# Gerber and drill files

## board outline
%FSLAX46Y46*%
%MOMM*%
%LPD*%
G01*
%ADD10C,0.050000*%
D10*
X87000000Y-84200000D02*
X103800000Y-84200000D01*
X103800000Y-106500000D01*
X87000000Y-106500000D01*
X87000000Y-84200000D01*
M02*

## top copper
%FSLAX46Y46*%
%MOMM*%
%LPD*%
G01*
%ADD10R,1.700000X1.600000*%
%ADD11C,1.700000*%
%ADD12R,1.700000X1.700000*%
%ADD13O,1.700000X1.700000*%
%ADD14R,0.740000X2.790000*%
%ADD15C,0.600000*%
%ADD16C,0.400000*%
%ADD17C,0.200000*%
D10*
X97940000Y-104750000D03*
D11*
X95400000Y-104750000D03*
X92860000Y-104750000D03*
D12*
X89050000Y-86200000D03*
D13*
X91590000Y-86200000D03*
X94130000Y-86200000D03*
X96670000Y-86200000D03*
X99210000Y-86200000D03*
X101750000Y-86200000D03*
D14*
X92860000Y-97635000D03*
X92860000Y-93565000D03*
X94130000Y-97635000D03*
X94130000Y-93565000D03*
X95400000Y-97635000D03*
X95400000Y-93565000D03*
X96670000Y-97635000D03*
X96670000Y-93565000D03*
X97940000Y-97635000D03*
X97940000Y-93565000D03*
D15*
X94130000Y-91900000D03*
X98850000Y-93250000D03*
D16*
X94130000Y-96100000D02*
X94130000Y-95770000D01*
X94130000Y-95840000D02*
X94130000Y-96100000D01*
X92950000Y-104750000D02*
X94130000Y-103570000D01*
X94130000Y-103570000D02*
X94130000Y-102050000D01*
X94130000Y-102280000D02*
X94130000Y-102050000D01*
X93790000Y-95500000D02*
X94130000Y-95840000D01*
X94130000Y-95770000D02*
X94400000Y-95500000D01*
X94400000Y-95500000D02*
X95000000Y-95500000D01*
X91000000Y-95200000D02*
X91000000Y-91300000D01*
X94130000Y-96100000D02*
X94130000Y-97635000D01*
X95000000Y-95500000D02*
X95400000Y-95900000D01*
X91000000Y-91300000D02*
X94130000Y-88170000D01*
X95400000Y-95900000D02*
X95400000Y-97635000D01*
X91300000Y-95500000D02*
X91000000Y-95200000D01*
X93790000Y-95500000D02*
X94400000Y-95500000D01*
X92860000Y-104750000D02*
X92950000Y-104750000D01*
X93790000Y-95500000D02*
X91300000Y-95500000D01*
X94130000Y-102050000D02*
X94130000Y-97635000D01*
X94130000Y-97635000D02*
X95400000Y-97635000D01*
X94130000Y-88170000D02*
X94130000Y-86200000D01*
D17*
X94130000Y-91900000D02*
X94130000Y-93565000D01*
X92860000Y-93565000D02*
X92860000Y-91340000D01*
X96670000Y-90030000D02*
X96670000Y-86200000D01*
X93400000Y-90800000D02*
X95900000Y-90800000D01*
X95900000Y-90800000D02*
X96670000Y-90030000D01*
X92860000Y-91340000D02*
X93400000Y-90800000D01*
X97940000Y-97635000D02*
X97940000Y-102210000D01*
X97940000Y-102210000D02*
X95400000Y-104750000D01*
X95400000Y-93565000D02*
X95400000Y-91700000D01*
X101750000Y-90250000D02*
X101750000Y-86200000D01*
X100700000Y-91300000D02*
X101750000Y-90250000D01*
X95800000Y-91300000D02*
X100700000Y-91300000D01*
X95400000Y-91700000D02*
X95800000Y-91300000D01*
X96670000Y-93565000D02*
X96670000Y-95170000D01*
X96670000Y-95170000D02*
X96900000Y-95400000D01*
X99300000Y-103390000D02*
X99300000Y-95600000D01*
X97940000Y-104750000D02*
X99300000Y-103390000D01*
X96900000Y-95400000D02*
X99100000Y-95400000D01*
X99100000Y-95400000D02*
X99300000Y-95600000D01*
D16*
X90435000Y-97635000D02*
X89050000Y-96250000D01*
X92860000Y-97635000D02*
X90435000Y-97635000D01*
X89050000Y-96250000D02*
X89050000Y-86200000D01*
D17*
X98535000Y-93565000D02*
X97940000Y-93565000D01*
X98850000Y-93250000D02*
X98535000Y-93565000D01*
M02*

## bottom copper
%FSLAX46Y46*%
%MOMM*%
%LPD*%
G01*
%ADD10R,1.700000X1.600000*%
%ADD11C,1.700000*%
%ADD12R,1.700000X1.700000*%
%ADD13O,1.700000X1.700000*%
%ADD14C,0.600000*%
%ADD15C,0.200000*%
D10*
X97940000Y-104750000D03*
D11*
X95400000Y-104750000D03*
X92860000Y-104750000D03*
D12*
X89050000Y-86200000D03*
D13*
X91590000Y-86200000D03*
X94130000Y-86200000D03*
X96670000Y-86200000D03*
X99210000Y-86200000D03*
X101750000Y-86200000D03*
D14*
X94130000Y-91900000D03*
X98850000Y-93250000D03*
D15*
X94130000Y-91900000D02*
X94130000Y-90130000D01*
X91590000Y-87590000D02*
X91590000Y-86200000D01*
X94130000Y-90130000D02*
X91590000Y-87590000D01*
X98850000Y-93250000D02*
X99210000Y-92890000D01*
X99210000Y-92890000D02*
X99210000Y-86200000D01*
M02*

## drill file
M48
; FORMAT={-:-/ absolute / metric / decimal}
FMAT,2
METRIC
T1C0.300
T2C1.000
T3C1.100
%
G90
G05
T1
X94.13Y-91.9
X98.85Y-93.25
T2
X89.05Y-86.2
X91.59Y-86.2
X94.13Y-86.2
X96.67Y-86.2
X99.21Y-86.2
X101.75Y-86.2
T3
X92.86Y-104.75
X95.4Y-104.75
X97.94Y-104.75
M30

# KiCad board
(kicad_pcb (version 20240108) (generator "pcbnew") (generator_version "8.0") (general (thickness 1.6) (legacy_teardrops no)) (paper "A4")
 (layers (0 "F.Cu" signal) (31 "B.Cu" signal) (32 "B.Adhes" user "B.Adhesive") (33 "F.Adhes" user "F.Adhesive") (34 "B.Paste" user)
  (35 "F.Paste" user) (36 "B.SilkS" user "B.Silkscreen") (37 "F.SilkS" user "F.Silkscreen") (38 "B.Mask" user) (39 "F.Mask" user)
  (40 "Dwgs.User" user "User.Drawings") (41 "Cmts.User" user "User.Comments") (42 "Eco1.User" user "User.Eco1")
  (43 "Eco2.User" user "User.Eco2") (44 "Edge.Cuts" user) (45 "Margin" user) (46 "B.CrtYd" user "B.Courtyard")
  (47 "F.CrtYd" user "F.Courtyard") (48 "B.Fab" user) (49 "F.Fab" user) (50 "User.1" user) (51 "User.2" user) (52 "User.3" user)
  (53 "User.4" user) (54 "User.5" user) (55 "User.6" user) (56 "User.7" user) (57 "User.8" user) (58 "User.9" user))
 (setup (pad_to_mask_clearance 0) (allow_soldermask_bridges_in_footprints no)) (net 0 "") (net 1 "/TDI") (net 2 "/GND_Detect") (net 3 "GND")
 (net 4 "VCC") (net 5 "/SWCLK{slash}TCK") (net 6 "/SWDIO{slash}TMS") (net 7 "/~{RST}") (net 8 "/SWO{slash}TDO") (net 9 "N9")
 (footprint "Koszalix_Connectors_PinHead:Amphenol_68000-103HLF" (layer "F.Cu") (at 95.4 104.75 180)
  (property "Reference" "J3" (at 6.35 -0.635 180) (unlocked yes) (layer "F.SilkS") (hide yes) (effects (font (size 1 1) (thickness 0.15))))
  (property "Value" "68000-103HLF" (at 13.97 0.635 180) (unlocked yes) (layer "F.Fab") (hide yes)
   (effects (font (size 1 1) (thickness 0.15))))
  (pad "1" thru_hole rect (at -2.54 0 180) (size 1.7 1.6) (drill 1.1) (layers "*.Cu" "*.Mask") (remove_unused_layers no) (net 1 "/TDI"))
  (pad "2" thru_hole circle (at 0 0 180) (size 1.7 1.7) (drill 1.1) (layers "*.Cu" "*.Mask") (remove_unused_layers no) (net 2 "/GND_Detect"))
  (pad "3" thru_hole circle (at 2.54 0 180) (size 1.7 1.7) (drill 1.1) (layers "*.Cu" "*.Mask") (remove_unused_layers no) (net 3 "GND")))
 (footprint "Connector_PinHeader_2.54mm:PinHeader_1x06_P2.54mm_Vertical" (layer "F.Cu") (at 89.05 86.2 90)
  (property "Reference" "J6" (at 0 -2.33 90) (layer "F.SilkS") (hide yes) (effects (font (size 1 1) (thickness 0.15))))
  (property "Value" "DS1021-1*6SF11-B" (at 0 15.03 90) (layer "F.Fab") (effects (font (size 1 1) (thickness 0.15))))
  (pad "1" thru_hole rect (at 0 0 90) (size 1.7 1.7) (drill 1) (layers "*.Cu" "*.Mask") (remove_unused_layers no) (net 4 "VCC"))
  (pad "2" thru_hole oval (at 0 2.54 90) (size 1.7 1.7) (drill 1) (layers "*.Cu" "*.Mask") (remove_unused_layers no)
   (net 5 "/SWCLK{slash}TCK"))
  (pad "3" thru_hole oval (at 0 5.08 90) (size 1.7 1.7) (drill 1) (layers "*.Cu" "*.Mask") (remove_unused_layers no) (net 3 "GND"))
  (pad "4" thru_hole oval (at 0 7.62 90) (size 1.7 1.7) (drill 1) (layers "*.Cu" "*.Mask") (remove_unused_layers no)
   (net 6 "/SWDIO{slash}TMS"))
  (pad "5" thru_hole oval (at 0 10.16 90) (size 1.7 1.7) (drill 1) (layers "*.Cu" "*.Mask") (remove_unused_layers no) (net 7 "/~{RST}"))
  (pad "6" thru_hole oval (at 0 12.7 90) (size 1.7 1.7) (drill 1) (layers "*.Cu" "*.Mask") (remove_unused_layers no)
   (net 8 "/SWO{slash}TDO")))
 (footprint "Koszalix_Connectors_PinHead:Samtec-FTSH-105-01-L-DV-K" (layer "F.Cu") (at 95.4 95.6)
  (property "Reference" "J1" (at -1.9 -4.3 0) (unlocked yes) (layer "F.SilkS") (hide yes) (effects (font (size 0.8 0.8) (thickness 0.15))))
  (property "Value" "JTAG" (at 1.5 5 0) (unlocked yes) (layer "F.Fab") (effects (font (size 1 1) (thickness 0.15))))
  (pad "1" smd rect (at -2.54 2.035) (size 0.74 2.79) (layers "F.Cu" "F.Paste" "F.Mask") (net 4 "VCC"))
  (pad "2" smd rect (at -2.54 -2.035) (size 0.74 2.79) (layers "F.Cu" "F.Paste" "F.Mask") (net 6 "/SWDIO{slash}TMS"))
  (pad "3" smd rect (at -1.27 2.035) (size 0.74 2.79) (layers "F.Cu" "F.Paste" "F.Mask") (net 3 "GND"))
  (pad "4" smd rect (at -1.27 -2.035) (size 0.74 2.79) (layers "F.Cu" "F.Paste" "F.Mask") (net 5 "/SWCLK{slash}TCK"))
  (pad "5" smd rect (at 0 2.035) (size 0.74 2.79) (layers "F.Cu" "F.Paste" "F.Mask") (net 3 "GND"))
  (pad "6" smd rect (at 0 -2.035) (size 0.74 2.79) (layers "F.Cu" "F.Paste" "F.Mask") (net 8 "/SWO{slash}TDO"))
  (pad "7" smd rect (at 1.27 2.035) (size 0.74 2.79) (layers "F.Cu" "F.Paste" "F.Mask") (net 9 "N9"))
  (pad "8" smd rect (at 1.27 -2.035) (size 0.74 2.79) (layers "F.Cu" "F.Paste" "F.Mask") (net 1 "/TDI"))
  (pad "9" smd rect (at 2.54 2.035) (size 0.74 2.79) (layers "F.Cu" "F.Paste" "F.Mask") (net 2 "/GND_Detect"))
  (pad "10" smd rect (at 2.54 -2.035) (size 0.74 2.79) (layers "F.Cu" "F.Paste" "F.Mask") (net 7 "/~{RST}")))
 (gr_rect (start 87 84.2) (end 103.8 106.5) (stroke (width 0.05) (type default)) (fill none) (layer "Edge.Cuts"))
 (segment (start 94.13 96.1) (end 94.13 95.77) (width 0.4) (layer "F.Cu") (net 3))
 (segment (start 94.13 95.84) (end 94.13 96.1) (width 0.4) (layer "F.Cu") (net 3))
 (segment (start 92.95 104.75) (end 94.13 103.57) (width 0.4) (layer "F.Cu") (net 3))
 (segment (start 94.13 103.57) (end 94.13 102.05) (width 0.4) (layer "F.Cu") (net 3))
 (segment (start 94.13 102.28) (end 94.13 102.05) (width 0.4) (layer "F.Cu") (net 3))
 (segment (start 93.79 95.5) (end 94.13 95.84) (width 0.4) (layer "F.Cu") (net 3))
 (segment (start 94.13 95.77) (end 94.4 95.5) (width 0.4) (layer "F.Cu") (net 3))
 (segment (start 94.4 95.5) (end 95 95.5) (width 0.4) (layer "F.Cu") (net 3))
 (segment (start 91 95.2) (end 91 91.3) (width 0.4) (layer "F.Cu") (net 3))
 (segment (start 94.13 96.1) (end 94.13 97.635) (width 0.4) (layer "F.Cu") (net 3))
 (segment (start 95 95.5) (end 95.4 95.9) (width 0.4) (layer "F.Cu") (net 3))
 (segment (start 91 91.3) (end 94.13 88.17) (width 0.4) (layer "F.Cu") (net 3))
 (segment (start 95.4 95.9) (end 95.4 97.635) (width 0.4) (layer "F.Cu") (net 3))
 (segment (start 91.3 95.5) (end 91 95.2) (width 0.4) (layer "F.Cu") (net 3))
 (segment (start 93.79 95.5) (end 94.4 95.5) (width 0.4) (layer "F.Cu") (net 3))
 (segment (start 92.86 104.75) (end 92.95 104.75) (width 0.4) (layer "F.Cu") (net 3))
 (segment (start 93.79 95.5) (end 91.3 95.5) (width 0.4) (layer "F.Cu") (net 3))
 (segment (start 94.13 102.05) (end 94.13 97.635) (width 0.4) (layer "F.Cu") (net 3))
 (segment (start 94.13 97.635) (end 95.4 97.635) (width 0.4) (layer "F.Cu") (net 3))
 (segment (start 94.13 88.17) (end 94.13 86.2) (width 0.4) (layer "F.Cu") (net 3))
 (segment (start 94.13 91.9) (end 94.13 93.565) (width 0.2) (layer "F.Cu") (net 5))
 (via (at 94.13 91.9) (size 0.6) (drill 0.3) (layers "F.Cu" "B.Cu") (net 5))
 (segment (start 94.13 91.9) (end 94.13 90.13) (width 0.2) (layer "B.Cu") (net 5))
 (segment (start 91.59 87.59) (end 91.59 86.2) (width 0.2) (layer "B.Cu") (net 5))
 (segment (start 94.13 90.13) (end 91.59 87.59) (width 0.2) (layer "B.Cu") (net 5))
 (segment (start 92.86 93.565) (end 92.86 91.34) (width 0.2) (layer "F.Cu") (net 6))
 (segment (start 96.67 90.03) (end 96.67 86.2) (width 0.2) (layer "F.Cu") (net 6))
 (segment (start 93.4 90.8) (end 95.9 90.8) (width 0.2) (layer "F.Cu") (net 6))
 (segment (start 95.9 90.8) (end 96.67 90.03) (width 0.2) (layer "F.Cu") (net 6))
 (segment (start 92.86 91.34) (end 93.4 90.8) (width 0.2) (layer "F.Cu") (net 6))
 (segment (start 97.94 97.635) (end 97.94 102.21) (width 0.2) (layer "F.Cu") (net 2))
 (segment (start 97.94 102.21) (end 95.4 104.75) (width 0.2) (layer "F.Cu") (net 2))
 (segment (start 95.4 93.565) (end 95.4 91.7) (width 0.2) (layer "F.Cu") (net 8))
 (segment (start 101.75 90.25) (end 101.75 86.2) (width 0.2) (layer "F.Cu") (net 8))
 (segment (start 100.7 91.3) (end 101.75 90.25) (width 0.2) (layer "F.Cu") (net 8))
 (segment (start 95.8 91.3) (end 100.7 91.3) (width 0.2) (layer "F.Cu") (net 8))
 (segment (start 95.4 91.7) (end 95.8 91.3) (width 0.2) (layer "F.Cu") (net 8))
 (segment (start 96.67 93.565) (end 96.67 95.17) (width 0.2) (layer "F.Cu") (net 1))
 (segment (start 96.67 95.17) (end 96.9 95.4) (width 0.2) (layer "F.Cu") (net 1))
 (segment (start 99.3 103.39) (end 99.3 95.6) (width 0.2) (layer "F.Cu") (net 1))
 (segment (start 97.94 104.75) (end 99.3 103.39) (width 0.2) (layer "F.Cu") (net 1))
 (segment (start 96.9 95.4) (end 99.1 95.4) (width 0.2) (layer "F.Cu") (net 1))
 (segment (start 99.1 95.4) (end 99.3 95.6) (width 0.2) (layer "F.Cu") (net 1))
 (segment (start 90.435 97.635) (end 89.05 96.25) (width 0.4) (layer "F.Cu") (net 4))
 (segment (start 92.86 97.635) (end 90.435 97.635) (width 0.4) (layer "F.Cu") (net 4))
 (segment (start 89.05 96.25) (end 89.05 86.2) (width 0.4) (layer "F.Cu") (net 4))
 (segment (start 98.535 93.565) (end 97.94 93.565) (width 0.2) (layer "F.Cu") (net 7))
 (segment (start 98.85 93.25) (end 98.535 93.565) (width 0.2) (layer "F.Cu") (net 7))
 (via (at 98.85 93.25) (size 0.6) (drill 0.3) (layers "F.Cu" "B.Cu") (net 7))
 (segment (start 98.85 93.25) (end 99.21 92.89) (width 0.2) (layer "B.Cu") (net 7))
 (segment (start 99.21 92.89) (end 99.21 86.2) (width 0.2) (layer "B.Cu") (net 7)))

